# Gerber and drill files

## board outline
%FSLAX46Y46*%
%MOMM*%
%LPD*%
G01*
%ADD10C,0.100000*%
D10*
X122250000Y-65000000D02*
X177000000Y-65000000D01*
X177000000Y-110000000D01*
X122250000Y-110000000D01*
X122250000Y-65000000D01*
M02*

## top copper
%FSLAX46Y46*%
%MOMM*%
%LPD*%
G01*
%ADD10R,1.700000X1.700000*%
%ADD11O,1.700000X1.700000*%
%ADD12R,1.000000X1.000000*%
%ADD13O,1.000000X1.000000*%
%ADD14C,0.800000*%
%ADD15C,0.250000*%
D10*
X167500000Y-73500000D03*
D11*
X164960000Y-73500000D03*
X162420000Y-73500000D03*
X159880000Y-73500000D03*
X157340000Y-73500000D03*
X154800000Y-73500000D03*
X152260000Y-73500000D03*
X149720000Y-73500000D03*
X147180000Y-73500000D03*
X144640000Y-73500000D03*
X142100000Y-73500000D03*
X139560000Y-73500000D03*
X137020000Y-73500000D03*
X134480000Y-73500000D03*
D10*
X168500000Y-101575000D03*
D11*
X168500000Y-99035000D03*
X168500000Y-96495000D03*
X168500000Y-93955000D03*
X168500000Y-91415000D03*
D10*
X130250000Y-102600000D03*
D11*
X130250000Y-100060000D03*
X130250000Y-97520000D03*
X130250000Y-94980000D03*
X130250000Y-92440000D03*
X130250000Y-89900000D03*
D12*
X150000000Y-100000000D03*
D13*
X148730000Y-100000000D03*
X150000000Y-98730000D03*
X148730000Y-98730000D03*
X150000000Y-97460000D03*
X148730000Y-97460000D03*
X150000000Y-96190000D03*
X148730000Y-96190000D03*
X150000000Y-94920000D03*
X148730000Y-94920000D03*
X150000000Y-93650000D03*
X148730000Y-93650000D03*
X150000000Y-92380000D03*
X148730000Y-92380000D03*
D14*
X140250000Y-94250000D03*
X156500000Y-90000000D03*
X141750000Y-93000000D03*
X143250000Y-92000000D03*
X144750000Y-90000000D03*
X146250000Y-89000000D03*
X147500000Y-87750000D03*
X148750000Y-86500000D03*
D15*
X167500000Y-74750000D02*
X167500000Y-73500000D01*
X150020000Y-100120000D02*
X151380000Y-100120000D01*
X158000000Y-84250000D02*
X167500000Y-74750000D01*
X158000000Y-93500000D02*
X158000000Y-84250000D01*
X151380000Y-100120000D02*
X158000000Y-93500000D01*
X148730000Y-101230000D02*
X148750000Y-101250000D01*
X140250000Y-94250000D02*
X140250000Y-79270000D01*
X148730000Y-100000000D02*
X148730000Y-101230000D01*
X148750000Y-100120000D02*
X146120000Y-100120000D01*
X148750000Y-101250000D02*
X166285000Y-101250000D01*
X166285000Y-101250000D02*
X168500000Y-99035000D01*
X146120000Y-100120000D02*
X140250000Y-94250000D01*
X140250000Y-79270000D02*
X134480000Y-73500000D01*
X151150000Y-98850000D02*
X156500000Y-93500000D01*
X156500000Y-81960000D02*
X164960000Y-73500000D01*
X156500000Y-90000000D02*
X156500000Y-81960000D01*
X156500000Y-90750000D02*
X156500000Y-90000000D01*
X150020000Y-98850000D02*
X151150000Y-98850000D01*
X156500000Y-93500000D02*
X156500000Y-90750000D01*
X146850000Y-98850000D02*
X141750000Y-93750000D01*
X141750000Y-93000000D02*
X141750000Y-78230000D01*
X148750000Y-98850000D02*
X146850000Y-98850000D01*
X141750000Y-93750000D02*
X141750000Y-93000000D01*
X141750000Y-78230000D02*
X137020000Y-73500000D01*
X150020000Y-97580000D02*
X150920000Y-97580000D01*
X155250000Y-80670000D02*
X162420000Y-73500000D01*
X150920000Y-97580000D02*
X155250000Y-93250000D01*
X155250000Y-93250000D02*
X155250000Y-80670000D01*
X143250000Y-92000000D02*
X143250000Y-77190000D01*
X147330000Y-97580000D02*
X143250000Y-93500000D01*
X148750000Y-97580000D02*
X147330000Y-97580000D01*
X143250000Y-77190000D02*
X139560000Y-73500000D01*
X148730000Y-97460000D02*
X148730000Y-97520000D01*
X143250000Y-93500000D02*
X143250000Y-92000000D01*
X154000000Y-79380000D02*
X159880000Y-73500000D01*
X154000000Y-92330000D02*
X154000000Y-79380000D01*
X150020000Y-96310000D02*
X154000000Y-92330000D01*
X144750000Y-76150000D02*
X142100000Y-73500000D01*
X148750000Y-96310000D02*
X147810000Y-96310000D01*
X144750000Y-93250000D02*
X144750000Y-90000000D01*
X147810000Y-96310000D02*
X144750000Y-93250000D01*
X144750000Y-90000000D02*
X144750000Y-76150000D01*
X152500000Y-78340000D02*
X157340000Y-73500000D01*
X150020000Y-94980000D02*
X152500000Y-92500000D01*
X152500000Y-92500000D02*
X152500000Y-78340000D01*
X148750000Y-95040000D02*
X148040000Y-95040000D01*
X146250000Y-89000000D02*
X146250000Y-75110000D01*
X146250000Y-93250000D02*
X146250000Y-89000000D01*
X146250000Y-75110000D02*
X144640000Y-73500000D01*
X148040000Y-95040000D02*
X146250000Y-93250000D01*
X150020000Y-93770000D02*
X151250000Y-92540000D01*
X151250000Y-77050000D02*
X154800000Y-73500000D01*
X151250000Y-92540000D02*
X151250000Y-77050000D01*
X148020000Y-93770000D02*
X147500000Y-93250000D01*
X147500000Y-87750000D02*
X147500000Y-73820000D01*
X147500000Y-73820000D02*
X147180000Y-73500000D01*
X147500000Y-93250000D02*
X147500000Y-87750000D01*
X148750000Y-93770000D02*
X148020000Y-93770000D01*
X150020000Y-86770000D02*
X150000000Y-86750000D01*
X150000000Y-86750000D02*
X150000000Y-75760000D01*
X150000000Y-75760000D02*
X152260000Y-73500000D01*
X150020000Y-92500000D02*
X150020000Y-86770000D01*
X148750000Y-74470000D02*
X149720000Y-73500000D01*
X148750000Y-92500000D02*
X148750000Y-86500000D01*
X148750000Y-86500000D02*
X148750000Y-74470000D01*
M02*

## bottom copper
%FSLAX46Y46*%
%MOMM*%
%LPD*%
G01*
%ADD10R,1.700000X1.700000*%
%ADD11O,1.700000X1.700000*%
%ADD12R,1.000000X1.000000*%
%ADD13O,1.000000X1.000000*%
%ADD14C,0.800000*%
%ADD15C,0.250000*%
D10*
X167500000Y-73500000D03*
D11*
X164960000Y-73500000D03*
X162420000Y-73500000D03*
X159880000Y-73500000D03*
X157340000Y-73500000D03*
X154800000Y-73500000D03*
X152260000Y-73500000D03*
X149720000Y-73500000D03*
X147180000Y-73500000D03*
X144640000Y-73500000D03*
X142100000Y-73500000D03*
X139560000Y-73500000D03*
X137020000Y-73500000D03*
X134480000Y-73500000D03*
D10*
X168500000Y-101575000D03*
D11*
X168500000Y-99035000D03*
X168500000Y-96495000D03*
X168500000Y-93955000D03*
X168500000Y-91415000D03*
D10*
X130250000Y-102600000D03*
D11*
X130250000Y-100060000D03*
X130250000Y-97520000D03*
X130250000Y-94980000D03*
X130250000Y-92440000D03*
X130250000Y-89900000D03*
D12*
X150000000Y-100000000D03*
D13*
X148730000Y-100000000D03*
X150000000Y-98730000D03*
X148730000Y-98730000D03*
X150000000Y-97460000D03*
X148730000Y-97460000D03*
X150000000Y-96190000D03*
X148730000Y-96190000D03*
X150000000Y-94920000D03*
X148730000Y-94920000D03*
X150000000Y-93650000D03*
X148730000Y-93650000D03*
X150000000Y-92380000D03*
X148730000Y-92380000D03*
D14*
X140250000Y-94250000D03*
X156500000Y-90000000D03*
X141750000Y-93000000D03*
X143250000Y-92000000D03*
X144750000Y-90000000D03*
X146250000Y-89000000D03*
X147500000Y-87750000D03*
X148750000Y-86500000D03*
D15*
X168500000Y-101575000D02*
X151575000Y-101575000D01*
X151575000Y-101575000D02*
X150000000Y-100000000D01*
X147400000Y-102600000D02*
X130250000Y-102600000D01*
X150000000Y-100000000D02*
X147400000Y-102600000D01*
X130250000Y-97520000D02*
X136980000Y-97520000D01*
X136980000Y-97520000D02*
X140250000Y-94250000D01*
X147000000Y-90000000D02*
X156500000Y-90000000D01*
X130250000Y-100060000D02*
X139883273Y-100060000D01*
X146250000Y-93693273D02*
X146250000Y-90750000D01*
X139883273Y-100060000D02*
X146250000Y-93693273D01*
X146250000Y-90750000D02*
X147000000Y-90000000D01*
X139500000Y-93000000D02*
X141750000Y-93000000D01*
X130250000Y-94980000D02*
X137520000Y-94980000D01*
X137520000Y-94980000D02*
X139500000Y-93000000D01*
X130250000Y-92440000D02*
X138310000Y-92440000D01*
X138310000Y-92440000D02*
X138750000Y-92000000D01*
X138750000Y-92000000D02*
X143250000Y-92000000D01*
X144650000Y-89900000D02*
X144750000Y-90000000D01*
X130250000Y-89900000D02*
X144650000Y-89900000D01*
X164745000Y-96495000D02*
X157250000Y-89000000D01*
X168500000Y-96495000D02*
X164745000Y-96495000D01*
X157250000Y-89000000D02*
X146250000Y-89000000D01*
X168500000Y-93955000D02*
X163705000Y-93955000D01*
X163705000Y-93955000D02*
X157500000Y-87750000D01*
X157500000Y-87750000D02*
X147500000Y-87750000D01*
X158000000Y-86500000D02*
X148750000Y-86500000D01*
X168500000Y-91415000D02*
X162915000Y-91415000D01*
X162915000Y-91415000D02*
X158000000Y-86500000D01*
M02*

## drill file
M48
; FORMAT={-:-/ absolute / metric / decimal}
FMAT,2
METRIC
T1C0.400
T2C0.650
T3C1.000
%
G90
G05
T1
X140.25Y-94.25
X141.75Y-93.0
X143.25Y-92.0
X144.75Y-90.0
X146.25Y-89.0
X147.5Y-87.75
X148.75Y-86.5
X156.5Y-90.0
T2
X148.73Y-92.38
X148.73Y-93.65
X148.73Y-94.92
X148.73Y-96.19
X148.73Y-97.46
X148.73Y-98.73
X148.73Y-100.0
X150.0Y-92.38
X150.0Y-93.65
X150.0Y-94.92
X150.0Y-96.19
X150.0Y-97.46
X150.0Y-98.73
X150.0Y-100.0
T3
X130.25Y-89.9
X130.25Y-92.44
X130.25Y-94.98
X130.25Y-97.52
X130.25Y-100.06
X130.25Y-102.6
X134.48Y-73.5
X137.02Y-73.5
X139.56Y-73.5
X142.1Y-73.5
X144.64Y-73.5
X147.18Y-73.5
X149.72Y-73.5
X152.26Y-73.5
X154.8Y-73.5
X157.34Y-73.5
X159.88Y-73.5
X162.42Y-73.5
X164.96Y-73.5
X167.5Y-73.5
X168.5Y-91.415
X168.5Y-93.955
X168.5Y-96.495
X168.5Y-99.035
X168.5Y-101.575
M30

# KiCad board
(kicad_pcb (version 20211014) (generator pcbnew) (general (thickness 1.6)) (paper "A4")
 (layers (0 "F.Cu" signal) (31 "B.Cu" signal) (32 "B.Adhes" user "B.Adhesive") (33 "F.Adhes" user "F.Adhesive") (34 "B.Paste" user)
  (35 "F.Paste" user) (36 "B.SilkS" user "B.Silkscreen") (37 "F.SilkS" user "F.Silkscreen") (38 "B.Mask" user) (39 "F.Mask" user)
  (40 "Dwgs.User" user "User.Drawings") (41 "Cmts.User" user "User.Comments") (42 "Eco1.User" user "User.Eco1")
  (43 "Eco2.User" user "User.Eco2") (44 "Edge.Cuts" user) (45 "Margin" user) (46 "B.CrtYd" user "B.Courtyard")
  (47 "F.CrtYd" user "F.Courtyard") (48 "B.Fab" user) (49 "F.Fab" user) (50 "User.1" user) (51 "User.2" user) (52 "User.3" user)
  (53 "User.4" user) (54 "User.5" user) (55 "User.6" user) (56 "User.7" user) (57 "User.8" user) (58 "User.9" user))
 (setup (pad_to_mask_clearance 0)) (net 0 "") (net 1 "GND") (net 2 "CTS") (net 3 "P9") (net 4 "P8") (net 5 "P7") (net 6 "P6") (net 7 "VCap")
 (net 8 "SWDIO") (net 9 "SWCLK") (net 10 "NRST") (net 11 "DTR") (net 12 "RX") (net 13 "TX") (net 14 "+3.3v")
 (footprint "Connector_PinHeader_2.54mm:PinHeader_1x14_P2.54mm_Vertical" (layer "F.Cu") (at 167.5 73.5 -90)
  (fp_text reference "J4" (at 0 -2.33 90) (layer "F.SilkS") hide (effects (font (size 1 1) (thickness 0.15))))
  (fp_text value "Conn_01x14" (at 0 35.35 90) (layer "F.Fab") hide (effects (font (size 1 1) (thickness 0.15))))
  (pad "1" thru_hole rect (at 0 0 270) (size 1.7 1.7) (drill 1) (layers *.Cu *.Mask) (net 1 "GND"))
  (pad "2" thru_hole oval (at 0 2.54 270) (size 1.7 1.7) (drill 1) (layers *.Cu *.Mask) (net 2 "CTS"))
  (pad "3" thru_hole oval (at 0 5.08 270) (size 1.7 1.7) (drill 1) (layers *.Cu *.Mask) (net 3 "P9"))
  (pad "4" thru_hole oval (at 0 7.62 270) (size 1.7 1.7) (drill 1) (layers *.Cu *.Mask) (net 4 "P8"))
  (pad "5" thru_hole oval (at 0 10.16 270) (size 1.7 1.7) (drill 1) (layers *.Cu *.Mask) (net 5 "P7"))
  (pad "6" thru_hole oval (at 0 12.7 270) (size 1.7 1.7) (drill 1) (layers *.Cu *.Mask) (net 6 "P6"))
  (pad "7" thru_hole oval (at 0 15.24 270) (size 1.7 1.7) (drill 1) (layers *.Cu *.Mask) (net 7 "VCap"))
  (pad "8" thru_hole oval (at 0 17.78 270) (size 1.7 1.7) (drill 1) (layers *.Cu *.Mask) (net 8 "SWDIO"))
  (pad "9" thru_hole oval (at 0 20.32 270) (size 1.7 1.7) (drill 1) (layers *.Cu *.Mask) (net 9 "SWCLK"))
  (pad "10" thru_hole oval (at 0 22.86 270) (size 1.7 1.7) (drill 1) (layers *.Cu *.Mask) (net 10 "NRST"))
  (pad "11" thru_hole oval (at 0 25.4 270) (size 1.7 1.7) (drill 1) (layers *.Cu *.Mask) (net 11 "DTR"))
  (pad "12" thru_hole oval (at 0 27.94 270) (size 1.7 1.7) (drill 1) (layers *.Cu *.Mask) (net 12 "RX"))
  (pad "13" thru_hole oval (at 0 30.48 270) (size 1.7 1.7) (drill 1) (layers *.Cu *.Mask) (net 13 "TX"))
  (pad "14" thru_hole oval (at 0 33.02 270) (size 1.7 1.7) (drill 1) (layers *.Cu *.Mask) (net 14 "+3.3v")))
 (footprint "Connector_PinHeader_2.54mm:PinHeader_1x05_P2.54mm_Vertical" (layer "F.Cu") (at 168.5 101.575 180)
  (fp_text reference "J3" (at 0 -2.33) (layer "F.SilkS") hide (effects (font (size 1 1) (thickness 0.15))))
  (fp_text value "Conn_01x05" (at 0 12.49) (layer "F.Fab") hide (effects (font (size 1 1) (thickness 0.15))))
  (pad "1" thru_hole rect (at 0 0 180) (size 1.7 1.7) (drill 1) (layers *.Cu *.Mask) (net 1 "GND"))
  (pad "2" thru_hole oval (at 0 2.54 180) (size 1.7 1.7) (drill 1) (layers *.Cu *.Mask) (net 14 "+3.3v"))
  (pad "3" thru_hole oval (at 0 5.08 180) (size 1.7 1.7) (drill 1) (layers *.Cu *.Mask) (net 10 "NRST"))
  (pad "4" thru_hole oval (at 0 7.62 180) (size 1.7 1.7) (drill 1) (layers *.Cu *.Mask) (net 9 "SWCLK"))
  (pad "5" thru_hole oval (at 0 10.16 180) (size 1.7 1.7) (drill 1) (layers *.Cu *.Mask) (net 8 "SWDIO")))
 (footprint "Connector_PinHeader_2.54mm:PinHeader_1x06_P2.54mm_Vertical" (layer "F.Cu") (at 130.25 102.6 180)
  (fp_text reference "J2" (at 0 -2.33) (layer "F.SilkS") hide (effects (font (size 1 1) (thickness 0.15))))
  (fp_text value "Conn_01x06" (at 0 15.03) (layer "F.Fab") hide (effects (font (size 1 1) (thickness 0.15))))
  (pad "1" thru_hole rect (at 0 0 180) (size 1.7 1.7) (drill 1) (layers *.Cu *.Mask) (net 1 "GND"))
  (pad "2" thru_hole oval (at 0 2.54 180) (size 1.7 1.7) (drill 1) (layers *.Cu *.Mask) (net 2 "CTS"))
  (pad "3" thru_hole oval (at 0 5.08 180) (size 1.7 1.7) (drill 1) (layers *.Cu *.Mask) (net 14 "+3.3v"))
  (pad "4" thru_hole oval (at 0 7.62 180) (size 1.7 1.7) (drill 1) (layers *.Cu *.Mask) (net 13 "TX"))
  (pad "5" thru_hole oval (at 0 10.16 180) (size 1.7 1.7) (drill 1) (layers *.Cu *.Mask) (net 12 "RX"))
  (pad "6" thru_hole oval (at 0 12.7 180) (size 1.7 1.7) (drill 1) (layers *.Cu *.Mask) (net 11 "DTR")))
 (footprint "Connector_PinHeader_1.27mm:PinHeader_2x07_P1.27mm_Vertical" (layer "F.Cu") (at 150 100 180)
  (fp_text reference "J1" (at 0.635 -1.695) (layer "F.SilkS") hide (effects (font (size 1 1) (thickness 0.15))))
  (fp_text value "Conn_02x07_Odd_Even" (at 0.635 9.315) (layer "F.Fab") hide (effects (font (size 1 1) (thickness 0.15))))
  (pad "1" thru_hole rect (at 0 0 180) (size 1 1) (drill 0.65) (layers *.Cu *.Mask) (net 1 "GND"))
  (pad "2" thru_hole oval (at 1.27 0 180) (size 1 1) (drill 0.65) (layers *.Cu *.Mask) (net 14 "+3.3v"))
  (pad "3" thru_hole oval (at 0 1.27 180) (size 1 1) (drill 0.65) (layers *.Cu *.Mask) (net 2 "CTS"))
  (pad "4" thru_hole oval (at 1.27 1.27 180) (size 1 1) (drill 0.65) (layers *.Cu *.Mask) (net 13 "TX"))
  (pad "5" thru_hole oval (at 0 2.54 180) (size 1 1) (drill 0.65) (layers *.Cu *.Mask) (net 3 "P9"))
  (pad "6" thru_hole oval (at 1.27 2.54 180) (size 1 1) (drill 0.65) (layers *.Cu *.Mask) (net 12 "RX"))
  (pad "7" thru_hole oval (at 0 3.81 180) (size 1 1) (drill 0.65) (layers *.Cu *.Mask) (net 4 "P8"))
  (pad "8" thru_hole oval (at 1.27 3.81 180) (size 1 1) (drill 0.65) (layers *.Cu *.Mask) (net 11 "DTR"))
  (pad "9" thru_hole oval (at 0 5.08 180) (size 1 1) (drill 0.65) (layers *.Cu *.Mask) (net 5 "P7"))
  (pad "10" thru_hole oval (at 1.27 5.08 180) (size 1 1) (drill 0.65) (layers *.Cu *.Mask) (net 10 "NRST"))
  (pad "11" thru_hole oval (at 0 6.35 180) (size 1 1) (drill 0.65) (layers *.Cu *.Mask) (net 6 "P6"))
  (pad "12" thru_hole oval (at 1.27 6.35 180) (size 1 1) (drill 0.65) (layers *.Cu *.Mask) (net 9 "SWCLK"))
  (pad "13" thru_hole oval (at 0 7.62 180) (size 1 1) (drill 0.65) (layers *.Cu *.Mask) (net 7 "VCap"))
  (pad "14" thru_hole oval (at 1.27 7.62 180) (size 1 1) (drill 0.65) (layers *.Cu *.Mask) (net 8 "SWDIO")))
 (gr_rect (start 177 110) (end 122.25 65) (layer "Edge.Cuts") (width 0.1) (fill none))
 (segment (start 167.5 74.75) (end 167.5 73.5) (width 0.25) (layer "F.Cu") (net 1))
 (segment (start 150.02 100.12) (end 151.38 100.12) (width 0.25) (layer "F.Cu") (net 1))
 (segment (start 158 84.25) (end 167.5 74.75) (width 0.25) (layer "F.Cu") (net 1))
 (segment (start 158 93.5) (end 158 84.25) (width 0.25) (layer "F.Cu") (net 1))
 (segment (start 151.38 100.12) (end 158 93.5) (width 0.25) (layer "F.Cu") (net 1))
 (segment (start 168.5 101.575) (end 151.575 101.575) (width 0.25) (layer "B.Cu") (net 1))
 (segment (start 151.575 101.575) (end 150 100) (width 0.25) (layer "B.Cu") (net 1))
 (segment (start 147.4 102.6) (end 130.25 102.6) (width 0.25) (layer "B.Cu") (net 1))
 (segment (start 150 100) (end 147.4 102.6) (width 0.25) (layer "B.Cu") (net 1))
 (segment (start 148.73 101.23) (end 148.75 101.25) (width 0.25) (layer "F.Cu") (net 14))
 (segment (start 140.25 94.25) (end 140.25 79.27) (width 0.25) (layer "F.Cu") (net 14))
 (segment (start 148.73 100) (end 148.73 101.23) (width 0.25) (layer "F.Cu") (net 14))
 (segment (start 148.75 100.12) (end 146.12 100.12) (width 0.25) (layer "F.Cu") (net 14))
 (segment (start 148.75 101.25) (end 166.285 101.25) (width 0.25) (layer "F.Cu") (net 14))
 (segment (start 166.285 101.25) (end 168.5 99.035) (width 0.25) (layer "F.Cu") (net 14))
 (segment (start 146.12 100.12) (end 140.25 94.25) (width 0.25) (layer "F.Cu") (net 14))
 (segment (start 140.25 79.27) (end 134.48 73.5) (width 0.25) (layer "F.Cu") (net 14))
 (via (at 140.25 94.25) (size 0.8) (drill 0.4) (layers "F.Cu" "B.Cu") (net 14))
 (segment (start 130.25 97.52) (end 136.98 97.52) (width 0.25) (layer "B.Cu") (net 14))
 (segment (start 136.98 97.52) (end 140.25 94.25) (width 0.25) (layer "B.Cu") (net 14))
 (segment (start 151.15 98.85) (end 156.5 93.5) (width 0.25) (layer "F.Cu") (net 2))
 (segment (start 156.5 81.96) (end 164.96 73.5) (width 0.25) (layer "F.Cu") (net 2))
 (segment (start 156.5 90) (end 156.5 81.96) (width 0.25) (layer "F.Cu") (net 2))
 (segment (start 156.5 90.75) (end 156.5 90) (width 0.25) (layer "F.Cu") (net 2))
 (segment (start 150.02 98.85) (end 151.15 98.85) (width 0.25) (layer "F.Cu") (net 2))
 (segment (start 156.5 93.5) (end 156.5 90.75) (width 0.25) (layer "F.Cu") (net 2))
 (via (at 156.5 90) (size 0.8) (drill 0.4) (layers "F.Cu" "B.Cu") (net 2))
 (segment (start 147 90) (end 156.5 90) (width 0.25) (layer "B.Cu") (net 2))
 (segment (start 130.25 100.06) (end 139.883273 100.06) (width 0.25) (layer "B.Cu") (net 2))
 (segment (start 146.25 93.693273) (end 146.25 90.75) (width 0.25) (layer "B.Cu") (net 2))
 (segment (start 139.883273 100.06) (end 146.25 93.693273) (width 0.25) (layer "B.Cu") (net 2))
 (segment (start 146.25 90.75) (end 147 90) (width 0.25) (layer "B.Cu") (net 2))
 (segment (start 146.85 98.85) (end 141.75 93.75) (width 0.25) (layer "F.Cu") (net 13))
 (segment (start 141.75 93) (end 141.75 78.23) (width 0.25) (layer "F.Cu") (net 13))
 (segment (start 148.75 98.85) (end 146.85 98.85) (width 0.25) (layer "F.Cu") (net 13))
 (segment (start 141.75 93.75) (end 141.75 93) (width 0.25) (layer "F.Cu") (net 13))
 (segment (start 141.75 78.23) (end 137.02 73.5) (width 0.25) (layer "F.Cu") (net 13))
 (via (at 141.75 93) (size 0.8) (drill 0.4) (layers "F.Cu" "B.Cu") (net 13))
 (segment (start 139.5 93) (end 141.75 93) (width 0.25) (layer "B.Cu") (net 13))
 (segment (start 130.25 94.98) (end 137.52 94.98) (width 0.25) (layer "B.Cu") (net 13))
 (segment (start 137.52 94.98) (end 139.5 93) (width 0.25) (layer "B.Cu") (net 13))
 (segment (start 150.02 97.58) (end 150.92 97.58) (width 0.25) (layer "F.Cu") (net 3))
 (segment (start 155.25 80.67) (end 162.42 73.5) (width 0.25) (layer "F.Cu") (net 3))
 (segment (start 150.92 97.58) (end 155.25 93.25) (width 0.25) (layer "F.Cu") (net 3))
 (segment (start 155.25 93.25) (end 155.25 80.67) (width 0.25) (layer "F.Cu") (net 3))
 (segment (start 143.25 92) (end 143.25 77.19) (width 0.25) (layer "F.Cu") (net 12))
 (segment (start 147.33 97.58) (end 143.25 93.5) (width 0.25) (layer "F.Cu") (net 12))
 (segment (start 148.75 97.58) (end 147.33 97.58) (width 0.25) (layer "F.Cu") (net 12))
 (segment (start 143.25 77.19) (end 139.56 73.5) (width 0.25) (layer "F.Cu") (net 12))
 (segment (start 148.73 97.46) (end 148.73 97.52) (width 0.25) (layer "F.Cu") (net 12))
 (segment (start 143.25 93.5) (end 143.25 92) (width 0.25) (layer "F.Cu") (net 12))
 (via (at 143.25 92) (size 0.8) (drill 0.4) (layers "F.Cu" "B.Cu") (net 12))
 (segment (start 130.25 92.44) (end 138.31 92.44) (width 0.25) (layer "B.Cu") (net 12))
 (segment (start 138.31 92.44) (end 138.75 92) (width 0.25) (layer "B.Cu") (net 12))
 (segment (start 138.75 92) (end 143.25 92) (width 0.25) (layer "B.Cu") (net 12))
 (segment (start 154 79.38) (end 159.88 73.5) (width 0.25) (layer "F.Cu") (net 4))
 (segment (start 154 92.33) (end 154 79.38) (width 0.25) (layer "F.Cu") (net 4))
 (segment (start 150.02 96.31) (end 154 92.33) (width 0.25) (layer "F.Cu") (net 4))
 (segment (start 144.75 76.15) (end 142.1 73.5) (width 0.25) (layer "F.Cu") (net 11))
 (segment (start 148.75 96.31) (end 147.81 96.31) (width 0.25) (layer "F.Cu") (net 11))
 (segment (start 144.75 93.25) (end 144.75 90) (width 0.25) (layer "F.Cu") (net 11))
 (segment (start 147.81 96.31) (end 144.75 93.25) (width 0.25) (layer "F.Cu") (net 11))
 (segment (start 144.75 90) (end 144.75 76.15) (width 0.25) (layer "F.Cu") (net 11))
 (via (at 144.75 90) (size 0.8) (drill 0.4) (layers "F.Cu" "B.Cu") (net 11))
 (segment (start 144.65 89.9) (end 144.75 90) (width 0.25) (layer "B.Cu") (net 11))
 (segment (start 130.25 89.9) (end 144.65 89.9) (width 0.25) (layer "B.Cu") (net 11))
 (segment (start 152.5 78.34) (end 157.34 73.5) (width 0.25) (layer "F.Cu") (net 5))
 (segment (start 150.02 94.98) (end 152.5 92.5) (width 0.25) (layer "F.Cu") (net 5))
 (segment (start 152.5 92.5) (end 152.5 78.34) (width 0.25) (layer "F.Cu") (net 5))
 (segment (start 148.75 95.04) (end 148.04 95.04) (width 0.25) (layer "F.Cu") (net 10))
 (segment (start 146.25 89) (end 146.25 75.11) (width 0.25) (layer "F.Cu") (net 10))
 (segment (start 146.25 93.25) (end 146.25 89) (width 0.25) (layer "F.Cu") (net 10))
 (segment (start 146.25 75.11) (end 144.64 73.5) (width 0.25) (layer "F.Cu") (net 10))
 (segment (start 148.04 95.04) (end 146.25 93.25) (width 0.25) (layer "F.Cu") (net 10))
 (via (at 146.25 89) (size 0.8) (drill 0.4) (layers "F.Cu" "B.Cu") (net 10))
 (segment (start 164.745 96.495) (end 157.25 89) (width 0.25) (layer "B.Cu") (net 10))
 (segment (start 168.5 96.495) (end 164.745 96.495) (width 0.25) (layer "B.Cu") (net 10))
 (segment (start 157.25 89) (end 146.25 89) (width 0.25) (layer "B.Cu") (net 10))
 (segment (start 150.02 93.77) (end 151.25 92.54) (width 0.25) (layer "F.Cu") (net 6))
 (segment (start 151.25 77.05) (end 154.8 73.5) (width 0.25) (layer "F.Cu") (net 6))
 (segment (start 151.25 92.54) (end 151.25 77.05) (width 0.25) (layer "F.Cu") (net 6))
 (segment (start 148.02 93.77) (end 147.5 93.25) (width 0.25) (layer "F.Cu") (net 9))
 (segment (start 147.5 87.75) (end 147.5 73.82) (width 0.25) (layer "F.Cu") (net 9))
 (segment (start 147.5 73.82) (end 147.18 73.5) (width 0.25) (layer "F.Cu") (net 9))
 (segment (start 147.5 93.25) (end 147.5 87.75) (width 0.25) (layer "F.Cu") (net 9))
 (segment (start 148.75 93.77) (end 148.02 93.77) (width 0.25) (layer "F.Cu") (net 9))
 (via (at 147.5 87.75) (size 0.8) (drill 0.4) (layers "F.Cu" "B.Cu") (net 9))
 (segment (start 168.5 93.955) (end 163.705 93.955) (width 0.25) (layer "B.Cu") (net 9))
 (segment (start 163.705 93.955) (end 157.5 87.75) (width 0.25) (layer "B.Cu") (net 9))
 (segment (start 157.5 87.75) (end 147.5 87.75) (width 0.25) (layer "B.Cu") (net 9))
 (segment (start 150.02 86.77) (end 150 86.75) (width 0.25) (layer "F.Cu") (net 7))
 (segment (start 150 86.75) (end 150 75.76) (width 0.25) (layer "F.Cu") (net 7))
 (segment (start 150 75.76) (end 152.26 73.5) (width 0.25) (layer "F.Cu") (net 7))
 (segment (start 150.02 92.5) (end 150.02 86.77) (width 0.25) (layer "F.Cu") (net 7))
 (segment (start 148.75 74.47) (end 149.72 73.5) (width 0.25) (layer "F.Cu") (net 8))
 (segment (start 148.75 92.5) (end 148.75 86.5) (width 0.25) (layer "F.Cu") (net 8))
 (segment (start 148.75 86.5) (end 148.75 74.47) (width 0.25) (layer "F.Cu") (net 8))
 (via (at 148.75 86.5) (size 0.8) (drill 0.4) (layers "F.Cu" "B.Cu") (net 8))
 (segment (start 158 86.5) (end 148.75 86.5) (width 0.25) (layer "B.Cu") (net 8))
 (segment (start 168.5 91.415) (end 162.915 91.415) (width 0.25) (layer "B.Cu") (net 8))
 (segment (start 162.915 91.415) (end 158 86.5) (width 0.25) (layer "B.Cu") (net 8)))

